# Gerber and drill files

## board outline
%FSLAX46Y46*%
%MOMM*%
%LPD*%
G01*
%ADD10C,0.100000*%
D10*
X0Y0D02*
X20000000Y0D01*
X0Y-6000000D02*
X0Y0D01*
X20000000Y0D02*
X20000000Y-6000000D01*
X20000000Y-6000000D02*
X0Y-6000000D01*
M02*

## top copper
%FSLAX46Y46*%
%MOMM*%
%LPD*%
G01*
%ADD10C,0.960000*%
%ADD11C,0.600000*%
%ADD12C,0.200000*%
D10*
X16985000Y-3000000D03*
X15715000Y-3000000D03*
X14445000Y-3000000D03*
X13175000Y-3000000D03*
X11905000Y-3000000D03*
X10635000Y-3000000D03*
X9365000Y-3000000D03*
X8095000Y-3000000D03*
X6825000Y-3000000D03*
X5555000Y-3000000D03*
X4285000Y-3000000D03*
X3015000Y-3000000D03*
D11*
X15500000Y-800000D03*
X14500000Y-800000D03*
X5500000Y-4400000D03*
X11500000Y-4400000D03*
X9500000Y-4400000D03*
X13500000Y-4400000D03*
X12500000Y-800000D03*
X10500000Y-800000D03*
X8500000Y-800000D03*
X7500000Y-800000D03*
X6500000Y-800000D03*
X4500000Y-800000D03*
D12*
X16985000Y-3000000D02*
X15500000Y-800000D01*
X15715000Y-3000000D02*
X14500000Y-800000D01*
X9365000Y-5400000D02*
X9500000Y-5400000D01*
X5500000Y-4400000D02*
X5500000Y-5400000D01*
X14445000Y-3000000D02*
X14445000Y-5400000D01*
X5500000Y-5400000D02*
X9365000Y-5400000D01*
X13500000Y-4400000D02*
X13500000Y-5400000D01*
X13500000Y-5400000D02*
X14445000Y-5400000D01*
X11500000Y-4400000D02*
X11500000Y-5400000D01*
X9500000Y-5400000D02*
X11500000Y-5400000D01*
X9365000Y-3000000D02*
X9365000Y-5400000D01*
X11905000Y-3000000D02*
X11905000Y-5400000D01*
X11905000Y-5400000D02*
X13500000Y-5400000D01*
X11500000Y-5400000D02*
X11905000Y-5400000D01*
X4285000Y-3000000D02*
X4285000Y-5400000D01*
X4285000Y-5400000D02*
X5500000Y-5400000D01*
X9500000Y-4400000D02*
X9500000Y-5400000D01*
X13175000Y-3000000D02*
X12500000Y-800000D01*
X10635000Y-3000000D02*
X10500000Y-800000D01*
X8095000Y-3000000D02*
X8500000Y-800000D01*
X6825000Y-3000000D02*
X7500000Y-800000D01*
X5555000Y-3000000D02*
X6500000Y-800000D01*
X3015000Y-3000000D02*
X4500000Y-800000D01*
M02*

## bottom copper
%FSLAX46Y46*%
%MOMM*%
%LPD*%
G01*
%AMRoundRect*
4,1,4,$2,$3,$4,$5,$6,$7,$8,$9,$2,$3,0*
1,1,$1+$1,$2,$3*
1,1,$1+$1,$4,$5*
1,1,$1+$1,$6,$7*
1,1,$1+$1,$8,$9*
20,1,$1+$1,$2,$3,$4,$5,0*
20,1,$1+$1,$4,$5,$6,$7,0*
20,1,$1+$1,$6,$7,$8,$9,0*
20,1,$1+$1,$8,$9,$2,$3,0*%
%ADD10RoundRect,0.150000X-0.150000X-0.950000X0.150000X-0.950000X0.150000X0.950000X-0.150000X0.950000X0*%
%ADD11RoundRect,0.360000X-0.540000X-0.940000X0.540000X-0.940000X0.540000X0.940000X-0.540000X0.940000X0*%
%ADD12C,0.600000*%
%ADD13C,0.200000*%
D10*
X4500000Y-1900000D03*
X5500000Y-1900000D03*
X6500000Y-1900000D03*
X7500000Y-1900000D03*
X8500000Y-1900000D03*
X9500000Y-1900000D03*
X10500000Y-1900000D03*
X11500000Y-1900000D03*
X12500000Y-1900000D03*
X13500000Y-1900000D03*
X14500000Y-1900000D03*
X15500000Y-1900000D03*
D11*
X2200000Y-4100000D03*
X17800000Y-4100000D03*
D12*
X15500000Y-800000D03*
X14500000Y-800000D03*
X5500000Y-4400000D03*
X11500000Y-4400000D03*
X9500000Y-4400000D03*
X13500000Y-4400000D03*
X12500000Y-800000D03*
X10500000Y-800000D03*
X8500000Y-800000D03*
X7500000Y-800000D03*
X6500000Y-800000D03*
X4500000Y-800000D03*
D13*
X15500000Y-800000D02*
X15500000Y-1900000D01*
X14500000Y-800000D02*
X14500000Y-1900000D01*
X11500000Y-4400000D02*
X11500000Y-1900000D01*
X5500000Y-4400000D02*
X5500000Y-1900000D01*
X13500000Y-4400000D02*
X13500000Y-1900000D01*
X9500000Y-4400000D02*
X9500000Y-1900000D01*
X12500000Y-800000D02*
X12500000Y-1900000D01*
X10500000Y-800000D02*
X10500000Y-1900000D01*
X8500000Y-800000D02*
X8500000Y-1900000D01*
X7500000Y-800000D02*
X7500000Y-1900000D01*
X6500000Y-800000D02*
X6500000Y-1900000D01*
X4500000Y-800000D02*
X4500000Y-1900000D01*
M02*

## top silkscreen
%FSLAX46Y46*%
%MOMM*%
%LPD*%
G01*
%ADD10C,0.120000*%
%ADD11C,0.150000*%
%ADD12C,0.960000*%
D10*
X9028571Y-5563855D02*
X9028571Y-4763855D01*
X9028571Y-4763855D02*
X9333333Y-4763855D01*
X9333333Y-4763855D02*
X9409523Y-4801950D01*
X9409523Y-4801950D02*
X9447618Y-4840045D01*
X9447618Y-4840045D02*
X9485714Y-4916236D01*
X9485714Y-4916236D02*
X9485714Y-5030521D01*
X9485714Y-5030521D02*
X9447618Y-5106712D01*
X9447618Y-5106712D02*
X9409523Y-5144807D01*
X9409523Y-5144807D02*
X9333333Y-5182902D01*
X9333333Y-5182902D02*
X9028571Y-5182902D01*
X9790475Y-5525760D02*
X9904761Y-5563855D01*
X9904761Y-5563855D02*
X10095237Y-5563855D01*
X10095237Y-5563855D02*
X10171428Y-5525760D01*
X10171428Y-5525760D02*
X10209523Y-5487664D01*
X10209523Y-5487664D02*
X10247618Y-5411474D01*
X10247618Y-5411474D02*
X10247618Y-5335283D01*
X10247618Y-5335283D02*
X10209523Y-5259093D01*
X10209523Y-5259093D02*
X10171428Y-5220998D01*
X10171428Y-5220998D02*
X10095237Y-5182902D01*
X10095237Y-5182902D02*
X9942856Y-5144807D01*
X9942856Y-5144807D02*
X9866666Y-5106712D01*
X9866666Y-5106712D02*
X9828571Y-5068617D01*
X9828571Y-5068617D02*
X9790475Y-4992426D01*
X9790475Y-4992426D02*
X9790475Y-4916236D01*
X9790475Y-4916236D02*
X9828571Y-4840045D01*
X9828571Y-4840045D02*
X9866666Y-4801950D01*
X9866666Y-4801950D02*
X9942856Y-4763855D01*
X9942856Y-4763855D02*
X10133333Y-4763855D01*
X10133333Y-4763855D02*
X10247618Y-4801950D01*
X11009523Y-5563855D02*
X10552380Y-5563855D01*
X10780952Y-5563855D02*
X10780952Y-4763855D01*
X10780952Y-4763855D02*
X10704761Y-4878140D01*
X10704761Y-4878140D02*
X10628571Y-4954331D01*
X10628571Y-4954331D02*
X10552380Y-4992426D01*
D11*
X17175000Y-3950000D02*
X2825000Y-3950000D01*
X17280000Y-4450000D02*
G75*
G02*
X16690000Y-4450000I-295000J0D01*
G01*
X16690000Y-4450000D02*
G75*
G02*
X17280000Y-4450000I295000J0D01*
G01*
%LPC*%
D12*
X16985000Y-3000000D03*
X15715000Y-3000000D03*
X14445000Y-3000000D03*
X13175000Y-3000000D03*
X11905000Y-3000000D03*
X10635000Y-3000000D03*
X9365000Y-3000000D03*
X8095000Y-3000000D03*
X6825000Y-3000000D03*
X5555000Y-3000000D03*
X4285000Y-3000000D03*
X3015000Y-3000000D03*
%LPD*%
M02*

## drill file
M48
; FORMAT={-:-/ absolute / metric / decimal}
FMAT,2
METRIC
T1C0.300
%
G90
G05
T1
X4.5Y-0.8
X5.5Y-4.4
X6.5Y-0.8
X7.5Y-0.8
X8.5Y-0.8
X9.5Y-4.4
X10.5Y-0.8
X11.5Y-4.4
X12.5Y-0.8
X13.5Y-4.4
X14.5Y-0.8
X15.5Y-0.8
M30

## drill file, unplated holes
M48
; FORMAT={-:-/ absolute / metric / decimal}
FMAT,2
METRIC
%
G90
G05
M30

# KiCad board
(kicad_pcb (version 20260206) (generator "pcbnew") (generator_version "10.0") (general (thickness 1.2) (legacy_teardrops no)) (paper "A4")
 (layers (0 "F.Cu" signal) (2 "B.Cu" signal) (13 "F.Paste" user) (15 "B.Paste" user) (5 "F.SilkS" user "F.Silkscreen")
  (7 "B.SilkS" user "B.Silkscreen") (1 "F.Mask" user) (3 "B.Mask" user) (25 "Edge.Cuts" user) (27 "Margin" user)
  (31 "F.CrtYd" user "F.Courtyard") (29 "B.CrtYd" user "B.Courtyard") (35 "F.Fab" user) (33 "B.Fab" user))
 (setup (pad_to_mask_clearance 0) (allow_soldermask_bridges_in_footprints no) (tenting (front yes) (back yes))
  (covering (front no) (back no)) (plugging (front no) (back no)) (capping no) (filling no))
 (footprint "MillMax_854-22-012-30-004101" (layer "F.Cu") (at 10 3 180)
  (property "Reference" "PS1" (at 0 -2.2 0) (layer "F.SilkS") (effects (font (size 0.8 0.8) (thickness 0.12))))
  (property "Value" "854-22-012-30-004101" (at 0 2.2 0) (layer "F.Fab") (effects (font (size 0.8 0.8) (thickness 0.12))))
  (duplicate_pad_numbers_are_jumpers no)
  (fp_line (start -7.175 -0.95) (end 7.175 -0.95) (stroke (width 0.15) (type solid)) (layer "F.SilkS"))
  (fp_circle (center -6.985 -1.45) (end -6.69 -1.45) (stroke (width 0.15) (type solid)) (fill no) (layer "F.SilkS"))
  (pad "1" smd circle (at -6.985 0) (size 0.96 0.96) (layers "F.Cu" "F.Mask" "F.Paste") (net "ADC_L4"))
  (pad "2" smd circle (at -5.715 0) (size 0.96 0.96) (layers "F.Cu" "F.Mask" "F.Paste") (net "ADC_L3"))
  (pad "3" smd circle (at -4.445 0) (size 0.96 0.96) (layers "F.Cu" "F.Mask" "F.Paste") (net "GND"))
  (pad "4" smd circle (at -3.175 0) (size 0.96 0.96) (layers "F.Cu" "F.Mask" "F.Paste") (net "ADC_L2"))
  (pad "5" smd circle (at -1.905 0) (size 0.96 0.96) (layers "F.Cu" "F.Mask" "F.Paste") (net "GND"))
  (pad "6" smd circle (at -0.635 0) (size 0.96 0.96) (layers "F.Cu" "F.Mask" "F.Paste") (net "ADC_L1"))
  (pad "7" smd circle (at 0.635 0) (size 0.96 0.96) (layers "F.Cu" "F.Mask" "F.Paste") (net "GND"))
  (pad "8" smd circle (at 1.905 0) (size 0.96 0.96) (layers "F.Cu" "F.Mask" "F.Paste") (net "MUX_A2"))
  (pad "9" smd circle (at 3.175 0) (size 0.96 0.96) (layers "F.Cu" "F.Mask" "F.Paste") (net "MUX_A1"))
  (pad "10" smd circle (at 4.445 0) (size 0.96 0.96) (layers "F.Cu" "F.Mask" "F.Paste") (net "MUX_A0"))
  (pad "11" smd circle (at 5.715 0) (size 0.96 0.96) (layers "F.Cu" "F.Mask" "F.Paste") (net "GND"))
  (pad "12" smd circle (at 6.985 0) (size 0.96 0.96) (layers "F.Cu" "F.Mask" "F.Paste") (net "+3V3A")))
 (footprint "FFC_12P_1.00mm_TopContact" (layer "B.Cu") (at 10 3)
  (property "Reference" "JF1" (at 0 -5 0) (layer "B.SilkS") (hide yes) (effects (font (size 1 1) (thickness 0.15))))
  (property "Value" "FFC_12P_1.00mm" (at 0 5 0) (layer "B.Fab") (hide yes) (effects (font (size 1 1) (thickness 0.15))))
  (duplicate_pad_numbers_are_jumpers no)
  (pad "1" smd roundrect (at -5.5 -1.1) (size 0.6 2.2) (layers "B.Cu" "B.Mask" "B.Paste") (roundrect_rratio 0.25) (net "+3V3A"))
  (pad "2" smd roundrect (at -4.5 -1.1) (size 0.6 2.2) (layers "B.Cu" "B.Mask" "B.Paste") (roundrect_rratio 0.25) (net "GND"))
  (pad "3" smd roundrect (at -3.5 -1.1) (size 0.6 2.2) (layers "B.Cu" "B.Mask" "B.Paste") (roundrect_rratio 0.25) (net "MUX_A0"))
  (pad "4" smd roundrect (at -2.5 -1.1) (size 0.6 2.2) (layers "B.Cu" "B.Mask" "B.Paste") (roundrect_rratio 0.25) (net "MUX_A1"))
  (pad "5" smd roundrect (at -1.5 -1.1) (size 0.6 2.2) (layers "B.Cu" "B.Mask" "B.Paste") (roundrect_rratio 0.25) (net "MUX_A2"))
  (pad "6" smd roundrect (at -0.5 -1.1) (size 0.6 2.2) (layers "B.Cu" "B.Mask" "B.Paste") (roundrect_rratio 0.25) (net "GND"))
  (pad "7" smd roundrect (at 0.5 -1.1) (size 0.6 2.2) (layers "B.Cu" "B.Mask" "B.Paste") (roundrect_rratio 0.25) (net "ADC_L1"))
  (pad "8" smd roundrect (at 1.5 -1.1) (size 0.6 2.2) (layers "B.Cu" "B.Mask" "B.Paste") (roundrect_rratio 0.25) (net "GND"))
  (pad "9" smd roundrect (at 2.5 -1.1) (size 0.6 2.2) (layers "B.Cu" "B.Mask" "B.Paste") (roundrect_rratio 0.25) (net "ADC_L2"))
  (pad "10" smd roundrect (at 3.5 -1.1) (size 0.6 2.2) (layers "B.Cu" "B.Mask" "B.Paste") (roundrect_rratio 0.25) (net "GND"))
  (pad "11" smd roundrect (at 4.5 -1.1) (size 0.6 2.2) (layers "B.Cu" "B.Mask" "B.Paste") (roundrect_rratio 0.25) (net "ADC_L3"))
  (pad "12" smd roundrect (at 5.5 -1.1) (size 0.6 2.2) (layers "B.Cu" "B.Mask" "B.Paste") (roundrect_rratio 0.25) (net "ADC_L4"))
  (pad "MP" smd roundrect (at -7.8 1.1) (size 1.8 2.6) (layers "B.Cu" "B.Mask" "B.Paste") (roundrect_rratio 0.2))
  (pad "MP" smd roundrect (at 7.8 1.1) (size 1.8 2.6) (layers "B.Cu" "B.Mask" "B.Paste") (roundrect_rratio 0.2)))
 (gr_line (start 0 0) (end 20 0) (stroke (width 0.1) (type solid)) (layer "Edge.Cuts"))
 (gr_line (start 0 6) (end 0 0) (stroke (width 0.1) (type solid)) (layer "Edge.Cuts"))
 (gr_line (start 20 0) (end 20 6) (stroke (width 0.1) (type solid)) (layer "Edge.Cuts"))
 (gr_line (start 20 6) (end 0 6) (stroke (width 0.1) (type solid)) (layer "Edge.Cuts"))
 (segment (start 16.985 3) (end 15.5 0.8) (width 0.2) (layer "F.Cu") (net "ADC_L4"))
 (via (at 15.5 0.8) (size 0.6) (drill 0.3) (layers "F.Cu" "B.Cu") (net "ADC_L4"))
 (segment (start 15.5 0.8) (end 15.5 1.9) (width 0.2) (layer "B.Cu") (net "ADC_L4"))
 (segment (start 15.715 3) (end 14.5 0.8) (width 0.2) (layer "F.Cu") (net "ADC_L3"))
 (via (at 14.5 0.8) (size 0.6) (drill 0.3) (layers "F.Cu" "B.Cu") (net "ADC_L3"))
 (segment (start 14.5 0.8) (end 14.5 1.9) (width 0.2) (layer "B.Cu") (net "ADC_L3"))
 (segment (start 9.365 5.4) (end 9.5 5.4) (width 0.2) (layer "F.Cu") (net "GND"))
 (segment (start 5.5 4.4) (end 5.5 5.4) (width 0.2) (layer "F.Cu") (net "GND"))
 (segment (start 14.445 3) (end 14.445 5.4) (width 0.2) (layer "F.Cu") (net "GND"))
 (segment (start 5.5 5.4) (end 9.365 5.4) (width 0.2) (layer "F.Cu") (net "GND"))
 (segment (start 13.5 4.4) (end 13.5 5.4) (width 0.2) (layer "F.Cu") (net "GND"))
 (segment (start 13.5 5.4) (end 14.445 5.4) (width 0.2) (layer "F.Cu") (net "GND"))
 (segment (start 11.5 4.4) (end 11.5 5.4) (width 0.2) (layer "F.Cu") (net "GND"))
 (segment (start 9.5 5.4) (end 11.5 5.4) (width 0.2) (layer "F.Cu") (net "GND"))
 (segment (start 9.365 3) (end 9.365 5.4) (width 0.2) (layer "F.Cu") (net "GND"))
 (segment (start 11.905 3) (end 11.905 5.4) (width 0.2) (layer "F.Cu") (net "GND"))
 (segment (start 11.905 5.4) (end 13.5 5.4) (width 0.2) (layer "F.Cu") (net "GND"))
 (segment (start 11.5 5.4) (end 11.905 5.4) (width 0.2) (layer "F.Cu") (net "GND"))
 (segment (start 4.285 3) (end 4.285 5.4) (width 0.2) (layer "F.Cu") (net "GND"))
 (segment (start 4.285 5.4) (end 5.5 5.4) (width 0.2) (layer "F.Cu") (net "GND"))
 (segment (start 9.5 4.4) (end 9.5 5.4) (width 0.2) (layer "F.Cu") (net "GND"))
 (via (at 5.5 4.4) (size 0.6) (drill 0.3) (layers "F.Cu" "B.Cu") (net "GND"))
 (via (at 11.5 4.4) (size 0.6) (drill 0.3) (layers "F.Cu" "B.Cu") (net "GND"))
 (via (at 9.5 4.4) (size 0.6) (drill 0.3) (layers "F.Cu" "B.Cu") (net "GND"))
 (via (at 13.5 4.4) (size 0.6) (drill 0.3) (layers "F.Cu" "B.Cu") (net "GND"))
 (segment (start 11.5 4.4) (end 11.5 1.9) (width 0.2) (layer "B.Cu") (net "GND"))
 (segment (start 5.5 4.4) (end 5.5 1.9) (width 0.2) (layer "B.Cu") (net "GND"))
 (segment (start 13.5 4.4) (end 13.5 1.9) (width 0.2) (layer "B.Cu") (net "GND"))
 (segment (start 9.5 4.4) (end 9.5 1.9) (width 0.2) (layer "B.Cu") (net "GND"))
 (segment (start 13.175 3) (end 12.5 0.8) (width 0.2) (layer "F.Cu") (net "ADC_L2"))
 (via (at 12.5 0.8) (size 0.6) (drill 0.3) (layers "F.Cu" "B.Cu") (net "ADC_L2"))
 (segment (start 12.5 0.8) (end 12.5 1.9) (width 0.2) (layer "B.Cu") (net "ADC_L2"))
 (segment (start 10.635 3) (end 10.5 0.8) (width 0.2) (layer "F.Cu") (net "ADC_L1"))
 (via (at 10.5 0.8) (size 0.6) (drill 0.3) (layers "F.Cu" "B.Cu") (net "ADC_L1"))
 (segment (start 10.5 0.8) (end 10.5 1.9) (width 0.2) (layer "B.Cu") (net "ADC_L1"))
 (segment (start 8.095 3) (end 8.5 0.8) (width 0.2) (layer "F.Cu") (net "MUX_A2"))
 (via (at 8.5 0.8) (size 0.6) (drill 0.3) (layers "F.Cu" "B.Cu") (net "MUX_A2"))
 (segment (start 8.5 0.8) (end 8.5 1.9) (width 0.2) (layer "B.Cu") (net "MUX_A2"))
 (segment (start 6.825 3) (end 7.5 0.8) (width 0.2) (layer "F.Cu") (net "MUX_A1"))
 (via (at 7.5 0.8) (size 0.6) (drill 0.3) (layers "F.Cu" "B.Cu") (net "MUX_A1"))
 (segment (start 7.5 0.8) (end 7.5 1.9) (width 0.2) (layer "B.Cu") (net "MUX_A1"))
 (segment (start 5.555 3) (end 6.5 0.8) (width 0.2) (layer "F.Cu") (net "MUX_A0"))
 (via (at 6.5 0.8) (size 0.6) (drill 0.3) (layers "F.Cu" "B.Cu") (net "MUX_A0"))
 (segment (start 6.5 0.8) (end 6.5 1.9) (width 0.2) (layer "B.Cu") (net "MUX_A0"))
 (segment (start 3.015 3) (end 4.5 0.8) (width 0.2) (layer "F.Cu") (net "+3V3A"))
 (via (at 4.5 0.8) (size 0.6) (drill 0.3) (layers "F.Cu" "B.Cu") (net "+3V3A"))
 (segment (start 4.5 0.8) (end 4.5 1.9) (width 0.2) (layer "B.Cu") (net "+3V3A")))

